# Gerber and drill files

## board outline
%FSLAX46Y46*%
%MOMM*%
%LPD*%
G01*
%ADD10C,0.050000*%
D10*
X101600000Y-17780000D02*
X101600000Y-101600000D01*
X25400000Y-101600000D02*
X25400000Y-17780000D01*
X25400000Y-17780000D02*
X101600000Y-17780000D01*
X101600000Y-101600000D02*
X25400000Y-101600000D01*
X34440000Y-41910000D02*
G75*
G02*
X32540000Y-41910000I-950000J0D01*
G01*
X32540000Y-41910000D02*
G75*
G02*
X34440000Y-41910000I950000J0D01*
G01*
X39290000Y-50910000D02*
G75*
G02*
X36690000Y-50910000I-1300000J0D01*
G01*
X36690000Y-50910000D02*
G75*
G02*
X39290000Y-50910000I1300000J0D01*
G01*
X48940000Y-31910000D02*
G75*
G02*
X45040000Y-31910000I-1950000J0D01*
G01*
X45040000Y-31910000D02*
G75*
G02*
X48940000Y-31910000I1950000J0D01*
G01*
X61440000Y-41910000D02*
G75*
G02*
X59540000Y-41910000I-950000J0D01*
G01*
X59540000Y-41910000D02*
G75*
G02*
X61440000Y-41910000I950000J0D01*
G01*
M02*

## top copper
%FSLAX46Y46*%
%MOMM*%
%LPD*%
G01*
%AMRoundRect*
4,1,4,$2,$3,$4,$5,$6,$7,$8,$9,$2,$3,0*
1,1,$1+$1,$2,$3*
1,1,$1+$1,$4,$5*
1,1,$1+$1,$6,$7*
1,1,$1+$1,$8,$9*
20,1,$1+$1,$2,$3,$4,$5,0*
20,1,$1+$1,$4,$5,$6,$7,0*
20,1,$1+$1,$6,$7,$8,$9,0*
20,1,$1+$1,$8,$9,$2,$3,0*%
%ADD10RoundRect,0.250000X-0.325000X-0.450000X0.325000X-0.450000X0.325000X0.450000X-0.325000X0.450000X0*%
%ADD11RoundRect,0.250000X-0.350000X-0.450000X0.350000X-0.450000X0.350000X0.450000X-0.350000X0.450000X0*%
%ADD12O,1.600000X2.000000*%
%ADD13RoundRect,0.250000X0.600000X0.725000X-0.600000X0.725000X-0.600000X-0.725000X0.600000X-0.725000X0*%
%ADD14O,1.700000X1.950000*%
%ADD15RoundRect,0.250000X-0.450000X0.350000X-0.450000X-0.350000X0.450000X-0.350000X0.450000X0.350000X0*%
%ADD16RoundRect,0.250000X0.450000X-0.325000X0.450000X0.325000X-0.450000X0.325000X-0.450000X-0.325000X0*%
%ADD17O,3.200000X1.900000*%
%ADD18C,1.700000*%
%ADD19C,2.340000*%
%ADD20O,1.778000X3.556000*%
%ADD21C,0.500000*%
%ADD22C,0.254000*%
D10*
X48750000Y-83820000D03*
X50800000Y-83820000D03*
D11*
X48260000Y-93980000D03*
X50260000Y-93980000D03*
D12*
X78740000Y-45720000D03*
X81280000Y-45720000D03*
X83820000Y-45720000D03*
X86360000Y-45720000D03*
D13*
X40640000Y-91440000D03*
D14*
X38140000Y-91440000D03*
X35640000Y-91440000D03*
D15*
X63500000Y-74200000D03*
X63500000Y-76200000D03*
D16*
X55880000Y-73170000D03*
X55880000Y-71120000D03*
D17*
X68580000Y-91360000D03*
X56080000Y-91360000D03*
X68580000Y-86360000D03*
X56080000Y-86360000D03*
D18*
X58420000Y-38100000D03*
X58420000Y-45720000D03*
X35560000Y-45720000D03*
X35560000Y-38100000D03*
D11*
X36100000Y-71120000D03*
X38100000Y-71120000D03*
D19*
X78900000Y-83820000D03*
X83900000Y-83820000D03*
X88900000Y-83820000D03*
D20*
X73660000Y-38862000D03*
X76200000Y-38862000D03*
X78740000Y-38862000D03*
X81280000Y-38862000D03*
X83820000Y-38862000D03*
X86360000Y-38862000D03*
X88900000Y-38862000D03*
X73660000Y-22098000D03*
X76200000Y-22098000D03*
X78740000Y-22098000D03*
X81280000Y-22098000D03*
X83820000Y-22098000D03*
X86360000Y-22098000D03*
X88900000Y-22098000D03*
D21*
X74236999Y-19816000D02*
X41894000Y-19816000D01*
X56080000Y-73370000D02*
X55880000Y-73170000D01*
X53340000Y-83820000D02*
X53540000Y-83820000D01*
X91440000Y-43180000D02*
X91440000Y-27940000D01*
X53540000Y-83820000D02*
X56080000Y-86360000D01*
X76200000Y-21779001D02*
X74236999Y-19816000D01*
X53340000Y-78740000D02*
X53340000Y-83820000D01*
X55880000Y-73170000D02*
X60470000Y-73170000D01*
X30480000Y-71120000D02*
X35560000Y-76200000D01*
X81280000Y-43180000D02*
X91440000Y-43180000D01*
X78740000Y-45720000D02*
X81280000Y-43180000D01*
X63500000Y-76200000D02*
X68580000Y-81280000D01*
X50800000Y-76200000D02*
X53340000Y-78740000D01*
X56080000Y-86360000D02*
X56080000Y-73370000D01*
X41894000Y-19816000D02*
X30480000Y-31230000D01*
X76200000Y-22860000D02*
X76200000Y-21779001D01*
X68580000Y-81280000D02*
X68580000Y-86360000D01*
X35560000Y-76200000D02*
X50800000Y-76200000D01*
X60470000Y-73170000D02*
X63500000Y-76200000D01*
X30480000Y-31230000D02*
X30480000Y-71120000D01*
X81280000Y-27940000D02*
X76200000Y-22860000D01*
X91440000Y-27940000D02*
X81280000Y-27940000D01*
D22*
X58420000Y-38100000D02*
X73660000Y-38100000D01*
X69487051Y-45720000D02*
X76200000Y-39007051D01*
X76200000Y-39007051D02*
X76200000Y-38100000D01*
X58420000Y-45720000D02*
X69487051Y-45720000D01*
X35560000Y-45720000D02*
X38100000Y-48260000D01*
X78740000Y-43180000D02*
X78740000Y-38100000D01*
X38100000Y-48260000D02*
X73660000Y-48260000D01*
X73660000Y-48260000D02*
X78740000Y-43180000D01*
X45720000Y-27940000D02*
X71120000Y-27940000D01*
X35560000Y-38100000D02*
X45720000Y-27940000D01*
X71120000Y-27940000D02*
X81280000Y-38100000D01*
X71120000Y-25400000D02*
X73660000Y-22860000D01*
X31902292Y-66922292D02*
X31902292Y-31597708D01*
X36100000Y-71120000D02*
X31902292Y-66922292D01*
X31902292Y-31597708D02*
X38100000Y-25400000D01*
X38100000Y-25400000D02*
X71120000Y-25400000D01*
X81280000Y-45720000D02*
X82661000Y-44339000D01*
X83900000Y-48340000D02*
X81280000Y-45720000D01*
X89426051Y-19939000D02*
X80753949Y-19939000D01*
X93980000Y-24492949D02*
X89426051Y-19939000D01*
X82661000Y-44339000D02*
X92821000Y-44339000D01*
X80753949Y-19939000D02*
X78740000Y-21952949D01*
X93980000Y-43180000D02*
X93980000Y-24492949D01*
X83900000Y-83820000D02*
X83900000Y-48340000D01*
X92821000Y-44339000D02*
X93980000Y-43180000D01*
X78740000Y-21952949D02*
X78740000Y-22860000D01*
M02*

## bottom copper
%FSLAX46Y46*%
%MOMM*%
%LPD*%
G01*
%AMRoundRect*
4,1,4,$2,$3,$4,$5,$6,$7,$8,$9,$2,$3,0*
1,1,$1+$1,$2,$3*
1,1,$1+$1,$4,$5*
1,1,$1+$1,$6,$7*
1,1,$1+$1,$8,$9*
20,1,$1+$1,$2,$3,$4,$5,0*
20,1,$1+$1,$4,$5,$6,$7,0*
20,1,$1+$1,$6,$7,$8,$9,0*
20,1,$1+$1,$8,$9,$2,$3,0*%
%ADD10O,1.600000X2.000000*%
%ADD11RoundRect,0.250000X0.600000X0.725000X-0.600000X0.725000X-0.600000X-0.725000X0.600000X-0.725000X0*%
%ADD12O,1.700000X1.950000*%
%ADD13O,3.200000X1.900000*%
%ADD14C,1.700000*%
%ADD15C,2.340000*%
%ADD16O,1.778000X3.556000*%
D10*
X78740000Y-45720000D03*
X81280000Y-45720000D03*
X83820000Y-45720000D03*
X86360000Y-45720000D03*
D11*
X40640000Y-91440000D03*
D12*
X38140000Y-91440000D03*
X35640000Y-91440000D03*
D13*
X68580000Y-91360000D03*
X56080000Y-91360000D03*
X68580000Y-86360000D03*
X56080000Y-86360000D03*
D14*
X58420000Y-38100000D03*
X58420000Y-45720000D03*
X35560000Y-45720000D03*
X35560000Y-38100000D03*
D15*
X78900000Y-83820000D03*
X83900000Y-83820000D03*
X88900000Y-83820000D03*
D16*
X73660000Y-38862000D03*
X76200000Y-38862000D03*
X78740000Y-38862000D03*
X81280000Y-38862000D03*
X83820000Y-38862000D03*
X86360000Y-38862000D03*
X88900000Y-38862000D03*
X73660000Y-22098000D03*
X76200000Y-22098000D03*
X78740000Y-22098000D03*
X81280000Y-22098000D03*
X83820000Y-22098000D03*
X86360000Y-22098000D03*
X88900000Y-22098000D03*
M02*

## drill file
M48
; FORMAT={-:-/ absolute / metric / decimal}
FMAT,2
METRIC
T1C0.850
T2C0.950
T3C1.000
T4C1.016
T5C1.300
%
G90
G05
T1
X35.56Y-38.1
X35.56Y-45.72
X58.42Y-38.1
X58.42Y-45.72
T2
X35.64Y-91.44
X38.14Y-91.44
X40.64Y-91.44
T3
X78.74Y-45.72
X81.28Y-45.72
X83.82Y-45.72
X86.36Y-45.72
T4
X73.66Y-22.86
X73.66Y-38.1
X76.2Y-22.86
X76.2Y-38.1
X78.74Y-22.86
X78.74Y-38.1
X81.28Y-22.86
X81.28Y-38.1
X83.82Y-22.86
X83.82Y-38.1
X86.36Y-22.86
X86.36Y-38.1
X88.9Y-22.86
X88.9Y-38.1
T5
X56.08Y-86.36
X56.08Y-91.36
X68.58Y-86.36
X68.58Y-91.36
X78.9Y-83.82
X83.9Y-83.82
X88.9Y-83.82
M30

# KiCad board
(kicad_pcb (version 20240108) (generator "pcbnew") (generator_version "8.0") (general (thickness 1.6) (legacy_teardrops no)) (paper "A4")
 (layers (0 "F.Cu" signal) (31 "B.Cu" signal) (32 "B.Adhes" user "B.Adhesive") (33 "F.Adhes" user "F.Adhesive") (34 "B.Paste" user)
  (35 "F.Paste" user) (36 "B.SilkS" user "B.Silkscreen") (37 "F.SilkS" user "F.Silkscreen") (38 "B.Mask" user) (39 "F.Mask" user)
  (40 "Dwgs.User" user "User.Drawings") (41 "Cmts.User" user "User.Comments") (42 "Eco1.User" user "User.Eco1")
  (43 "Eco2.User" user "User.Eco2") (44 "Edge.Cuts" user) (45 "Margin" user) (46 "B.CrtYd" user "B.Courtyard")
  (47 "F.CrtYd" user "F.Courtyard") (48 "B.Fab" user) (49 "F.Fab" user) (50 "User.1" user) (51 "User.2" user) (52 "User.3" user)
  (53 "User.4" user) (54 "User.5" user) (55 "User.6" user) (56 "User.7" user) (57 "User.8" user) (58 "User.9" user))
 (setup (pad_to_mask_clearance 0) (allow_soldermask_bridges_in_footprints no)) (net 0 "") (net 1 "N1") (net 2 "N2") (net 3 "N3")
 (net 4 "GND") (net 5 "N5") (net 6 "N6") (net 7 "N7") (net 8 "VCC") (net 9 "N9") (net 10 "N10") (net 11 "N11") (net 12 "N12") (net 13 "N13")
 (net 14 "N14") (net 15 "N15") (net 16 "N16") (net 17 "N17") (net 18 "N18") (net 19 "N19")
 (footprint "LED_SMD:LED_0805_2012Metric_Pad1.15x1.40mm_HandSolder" (layer "F.Cu") (at 49.775 83.82)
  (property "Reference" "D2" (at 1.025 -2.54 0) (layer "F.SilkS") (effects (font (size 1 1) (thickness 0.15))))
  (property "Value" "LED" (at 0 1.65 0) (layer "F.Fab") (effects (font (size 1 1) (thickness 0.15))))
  (pad "1" smd roundrect (at -1.025 0) (size 1.15 1.4) (layers "F.Cu" "F.Paste" "F.Mask") (roundrect_rratio 0.217391) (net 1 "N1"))
  (pad "2" smd roundrect (at 1.025 0) (size 1.15 1.4) (layers "F.Cu" "F.Paste" "F.Mask") (roundrect_rratio 0.217391) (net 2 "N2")))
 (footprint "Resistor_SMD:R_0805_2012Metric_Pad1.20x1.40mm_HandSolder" (layer "F.Cu") (at 49.26 93.98)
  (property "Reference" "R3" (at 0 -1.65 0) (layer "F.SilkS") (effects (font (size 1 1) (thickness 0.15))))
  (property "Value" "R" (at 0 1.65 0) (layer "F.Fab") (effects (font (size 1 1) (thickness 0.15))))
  (pad "1" smd roundrect (at -1 0) (size 1.2 1.4) (layers "F.Cu" "F.Paste" "F.Mask") (roundrect_rratio 0.208333) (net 1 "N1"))
  (pad "2" smd roundrect (at 1 0) (size 1.2 1.4) (layers "F.Cu" "F.Paste" "F.Mask") (roundrect_rratio 0.208333) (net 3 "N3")))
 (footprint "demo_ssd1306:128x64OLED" (layer "F.Cu") (at 82.36 56.32)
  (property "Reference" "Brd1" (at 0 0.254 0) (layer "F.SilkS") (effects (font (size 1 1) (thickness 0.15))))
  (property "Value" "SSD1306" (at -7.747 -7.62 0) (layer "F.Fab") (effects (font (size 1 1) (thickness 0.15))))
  (pad "1" thru_hole oval (at -3.62 -10.6 90) (size 2 1.6) (drill 1) (layers "*.Cu" "*.Mask") (remove_unused_layers no) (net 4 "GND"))
  (pad "2" thru_hole oval (at -1.08 -10.6 90) (size 2 1.6) (drill 1) (layers "*.Cu" "*.Mask") (remove_unused_layers no) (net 2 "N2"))
  (pad "3" thru_hole oval (at 1.46 -10.6 90) (size 2 1.6) (drill 1) (layers "*.Cu" "*.Mask") (remove_unused_layers no) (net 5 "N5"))
  (pad "4" thru_hole oval (at 4 -10.6 90) (size 2 1.6) (drill 1) (layers "*.Cu" "*.Mask") (remove_unused_layers no) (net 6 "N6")))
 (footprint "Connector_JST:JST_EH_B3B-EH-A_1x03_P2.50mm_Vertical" (layer "F.Cu") (at 40.64 91.44 180)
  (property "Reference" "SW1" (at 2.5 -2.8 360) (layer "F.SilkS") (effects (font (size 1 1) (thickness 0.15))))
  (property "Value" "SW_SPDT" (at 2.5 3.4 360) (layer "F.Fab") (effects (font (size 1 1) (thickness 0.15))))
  (pad "1" thru_hole roundrect (at 0 0 180) (size 1.7 1.95) (drill 0.95) (layers "*.Cu" "*.Mask") (remove_unused_layers no)
   (roundrect_rratio 0.147059) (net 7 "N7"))
  (pad "2" thru_hole oval (at 2.5 0 180) (size 1.7 1.95) (drill 0.95) (layers "*.Cu" "*.Mask") (remove_unused_layers no) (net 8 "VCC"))
  (pad "3" thru_hole oval (at 5 0 180) (size 1.7 1.95) (drill 0.95) (layers "*.Cu" "*.Mask") (remove_unused_layers no) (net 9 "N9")))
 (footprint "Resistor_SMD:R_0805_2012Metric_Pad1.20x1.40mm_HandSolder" (layer "F.Cu") (at 63.5 75.2 -90)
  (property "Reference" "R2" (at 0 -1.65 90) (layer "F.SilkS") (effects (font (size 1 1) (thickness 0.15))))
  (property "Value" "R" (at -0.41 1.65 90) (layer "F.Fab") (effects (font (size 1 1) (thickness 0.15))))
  (pad "1" smd roundrect (at -1 0 270) (size 1.2 1.4) (layers "F.Cu" "F.Paste" "F.Mask") (roundrect_rratio 0.208333) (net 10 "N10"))
  (pad "2" smd roundrect (at 1 0 270) (size 1.2 1.4) (layers "F.Cu" "F.Paste" "F.Mask") (roundrect_rratio 0.208333) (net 4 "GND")))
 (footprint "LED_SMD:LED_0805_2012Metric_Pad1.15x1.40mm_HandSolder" (layer "F.Cu") (at 55.88 72.145 90)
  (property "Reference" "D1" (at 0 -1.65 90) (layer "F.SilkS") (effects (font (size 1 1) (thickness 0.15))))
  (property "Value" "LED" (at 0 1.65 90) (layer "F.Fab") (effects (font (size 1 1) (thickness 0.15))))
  (pad "1" smd roundrect (at -1.025 0 90) (size 1.15 1.4) (layers "F.Cu" "F.Paste" "F.Mask") (roundrect_rratio 0.217391) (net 4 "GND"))
  (pad "2" smd roundrect (at 1.025 0 90) (size 1.15 1.4) (layers "F.Cu" "F.Paste" "F.Mask") (roundrect_rratio 0.217391) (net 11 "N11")))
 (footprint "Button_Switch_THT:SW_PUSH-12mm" (layer "F.Cu") (at 68.58 91.36 180)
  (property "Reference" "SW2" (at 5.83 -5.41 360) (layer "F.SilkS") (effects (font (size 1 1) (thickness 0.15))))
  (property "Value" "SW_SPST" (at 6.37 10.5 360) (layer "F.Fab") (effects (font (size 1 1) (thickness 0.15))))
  (pad "1" thru_hole oval (at 0 0 180) (size 3.2 1.9) (drill 1.3) (layers "*.Cu" "*.Mask") (remove_unused_layers no) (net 3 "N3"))
  (pad "1" thru_hole oval (at 12.5 0 180) (size 3.2 1.9) (drill 1.3) (layers "*.Cu" "*.Mask") (remove_unused_layers no) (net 3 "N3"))
  (pad "2" thru_hole oval (at 0 5 180) (size 3.2 1.9) (drill 1.3) (layers "*.Cu" "*.Mask") (remove_unused_layers no) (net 4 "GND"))
  (pad "2" thru_hole oval (at 12.5 5 180) (size 3.2 1.9) (drill 1.3) (layers "*.Cu" "*.Mask") (remove_unused_layers no) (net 4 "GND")))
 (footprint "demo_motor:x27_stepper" (layer "F.Cu") (at 49.53 52.07)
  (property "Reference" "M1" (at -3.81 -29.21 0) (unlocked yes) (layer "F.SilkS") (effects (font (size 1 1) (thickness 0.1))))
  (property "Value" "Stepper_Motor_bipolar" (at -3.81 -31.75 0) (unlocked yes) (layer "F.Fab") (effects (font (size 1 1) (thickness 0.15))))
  (fp_circle (center -16.04 -10.16) (end -15.09 -10.16) (stroke (width 0.05) (type default)) (fill none) (layer "Edge.Cuts"))
  (fp_circle (center -11.54 -1.16) (end -10.24 -1.16) (stroke (width 0.05) (type default)) (fill none) (layer "Edge.Cuts"))
  (fp_circle (center -2.54 -20.16) (end -0.59 -20.16) (stroke (width 0.05) (type default)) (fill none) (layer "Edge.Cuts"))
  (fp_circle (center 10.96 -10.16) (end 11.91 -10.16) (stroke (width 0.05) (type default)) (fill none) (layer "Edge.Cuts"))
  (pad "1" thru_hole circle (at 8.89 -13.97) (size 1.7 1.7) (drill 0.85) (layers "*.Cu" "*.Mask") (remove_unused_layers no) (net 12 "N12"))
  (pad "2" thru_hole circle (at 8.89 -6.35) (size 1.7 1.7) (drill 0.85) (layers "*.Cu" "*.Mask") (remove_unused_layers no) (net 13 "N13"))
  (pad "3" thru_hole circle (at -13.97 -6.35) (size 1.7 1.7) (drill 0.85) (layers "*.Cu" "*.Mask") (remove_unused_layers no) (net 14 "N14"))
  (pad "4" thru_hole circle (at -13.97 -13.97) (size 1.7 1.7) (drill 0.85) (layers "*.Cu" "*.Mask") (remove_unused_layers no) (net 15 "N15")))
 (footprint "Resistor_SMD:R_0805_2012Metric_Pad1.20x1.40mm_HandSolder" (layer "F.Cu") (at 37.1 71.12)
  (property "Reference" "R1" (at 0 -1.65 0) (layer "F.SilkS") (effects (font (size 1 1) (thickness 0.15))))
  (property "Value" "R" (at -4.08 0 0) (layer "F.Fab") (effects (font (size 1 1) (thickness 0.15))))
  (pad "1" smd roundrect (at -1 0) (size 1.2 1.4) (layers "F.Cu" "F.Paste" "F.Mask") (roundrect_rratio 0.208333) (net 9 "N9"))
  (pad "2" smd roundrect (at 1 0) (size 1.2 1.4) (layers "F.Cu" "F.Paste" "F.Mask") (roundrect_rratio 0.208333) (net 11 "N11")))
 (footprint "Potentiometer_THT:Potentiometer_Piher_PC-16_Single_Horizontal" (layer "F.Cu") (at 78.9 83.82 -90)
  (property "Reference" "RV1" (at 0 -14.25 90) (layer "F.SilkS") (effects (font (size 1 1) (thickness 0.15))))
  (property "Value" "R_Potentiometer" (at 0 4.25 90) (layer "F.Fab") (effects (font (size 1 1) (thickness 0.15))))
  (pad "1" thru_hole circle (at 0 0 270) (size 2.34 2.34) (drill 1.3) (layers "*.Cu" "*.Mask") (remove_unused_layers no) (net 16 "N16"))
  (pad "2" thru_hole circle (at 0 -5 270) (size 2.34 2.34) (drill 1.3) (layers "*.Cu" "*.Mask") (remove_unused_layers no) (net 2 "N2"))
  (pad "3" thru_hole circle (at 0 -10 270) (size 2.34 2.34) (drill 1.3) (layers "*.Cu" "*.Mask") (remove_unused_layers no) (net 10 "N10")))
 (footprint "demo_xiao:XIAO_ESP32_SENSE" (layer "F.Cu") (at 81.28 30.48 90)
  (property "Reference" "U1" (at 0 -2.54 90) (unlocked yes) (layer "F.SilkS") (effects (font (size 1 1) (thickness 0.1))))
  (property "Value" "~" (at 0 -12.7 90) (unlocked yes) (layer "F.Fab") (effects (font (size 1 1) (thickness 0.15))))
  (pad "1" thru_hole oval (at -7.62 -7.62 90) (size 3.556 1.778) (drill 1.016 (offset -0.762 0)) (layers "*.Cu" "*.Mask")
   (remove_unused_layers no) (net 12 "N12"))
  (pad "2" thru_hole oval (at -7.62 -5.08 90) (size 3.556 1.778) (drill 1.016 (offset -0.762 0)) (layers "*.Cu" "*.Mask")
   (remove_unused_layers no) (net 13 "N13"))
  (pad "3" thru_hole oval (at -7.62 -2.54 90) (size 3.556 1.778) (drill 1.016 (offset -0.762 0)) (layers "*.Cu" "*.Mask")
   (remove_unused_layers no) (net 14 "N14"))
  (pad "4" thru_hole oval (at -7.62 0 90) (size 3.556 1.778) (drill 1.016 (offset -0.762 0)) (layers "*.Cu" "*.Mask")
   (remove_unused_layers no) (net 15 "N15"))
  (pad "5" thru_hole oval (at -7.62 2.54 90) (size 3.556 1.778) (drill 1.016 (offset -0.762 0)) (layers "*.Cu" "*.Mask")
   (remove_unused_layers no) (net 6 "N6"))
  (pad "6" thru_hole oval (at -7.62 5.08 90) (size 3.556 1.778) (drill 1.016 (offset -0.762 0)) (layers "*.Cu" "*.Mask")
   (remove_unused_layers no) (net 5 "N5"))
  (pad "7" thru_hole oval (at -7.62 7.62 90) (size 3.556 1.778) (drill 1.016 (offset -0.762 0)) (layers "*.Cu" "*.Mask")
   (remove_unused_layers no) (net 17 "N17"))
  (pad "8" thru_hole oval (at 7.62 -7.62 90) (size 3.556 1.778) (drill 1.016 (offset 0.762 0)) (layers "*.Cu" "*.Mask")
   (remove_unused_layers no) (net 9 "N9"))
  (pad "9" thru_hole oval (at 7.62 -5.08 90) (size 3.556 1.778) (drill 1.016 (offset 0.762 0)) (layers "*.Cu" "*.Mask")
   (remove_unused_layers no) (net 4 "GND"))
  (pad "10" thru_hole oval (at 7.62 -2.54 90) (size 3.556 1.778) (drill 1.016 (offset 0.762 0)) (layers "*.Cu" "*.Mask")
   (remove_unused_layers no) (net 2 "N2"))
  (pad "11" thru_hole oval (at 7.62 0 90) (size 3.556 1.778) (drill 1.016 (offset 0.762 0)) (layers "*.Cu" "*.Mask")
   (remove_unused_layers no) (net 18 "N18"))
  (pad "12" thru_hole oval (at 7.62 2.54 90) (size 3.556 1.778) (drill 1.016 (offset 0.762 0)) (layers "*.Cu" "*.Mask")
   (remove_unused_layers no) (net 10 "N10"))
  (pad "13" thru_hole oval (at 7.62 5.08 90) (size 3.556 1.778) (drill 1.016 (offset 0.762 0)) (layers "*.Cu" "*.Mask")
   (remove_unused_layers no) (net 3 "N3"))
  (pad "14" thru_hole oval (at 7.62 7.62 90) (size 3.556 1.778) (drill 1.016 (offset 0.762 0)) (layers "*.Cu" "*.Mask")
   (remove_unused_layers no) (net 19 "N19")))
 (gr_line (start 101.6 17.78) (end 101.6 101.6) (stroke (width 0.05) (type default)) (layer "Edge.Cuts"))
 (gr_line (start 25.4 101.6) (end 25.4 17.78) (stroke (width 0.05) (type default)) (layer "Edge.Cuts"))
 (gr_line (start 25.4 17.78) (end 101.6 17.78) (stroke (width 0.05) (type default)) (layer "Edge.Cuts"))
 (gr_line (start 101.6 101.6) (end 25.4 101.6) (stroke (width 0.05) (type default)) (layer "Edge.Cuts"))
 (segment (start 74.236999 19.816) (end 41.894 19.816) (width 0.5) (layer "F.Cu") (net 4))
 (segment (start 56.08 73.37) (end 55.88 73.17) (width 0.5) (layer "F.Cu") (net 4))
 (segment (start 53.34 83.82) (end 53.54 83.82) (width 0.5) (layer "F.Cu") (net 4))
 (segment (start 91.44 43.18) (end 91.44 27.94) (width 0.5) (layer "F.Cu") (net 4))
 (segment (start 53.54 83.82) (end 56.08 86.36) (width 0.5) (layer "F.Cu") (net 4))
 (segment (start 76.2 21.779001) (end 74.236999 19.816) (width 0.5) (layer "F.Cu") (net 4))
 (segment (start 53.34 78.74) (end 53.34 83.82) (width 0.5) (layer "F.Cu") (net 4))
 (segment (start 55.88 73.17) (end 60.47 73.17) (width 0.5) (layer "F.Cu") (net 4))
 (segment (start 30.48 71.12) (end 35.56 76.2) (width 0.5) (layer "F.Cu") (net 4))
 (segment (start 81.28 43.18) (end 91.44 43.18) (width 0.5) (layer "F.Cu") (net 4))
 (segment (start 78.74 45.72) (end 81.28 43.18) (width 0.5) (layer "F.Cu") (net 4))
 (segment (start 63.5 76.2) (end 68.58 81.28) (width 0.5) (layer "F.Cu") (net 4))
 (segment (start 50.8 76.2) (end 53.34 78.74) (width 0.5) (layer "F.Cu") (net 4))
 (segment (start 56.08 86.36) (end 56.08 73.37) (width 0.5) (layer "F.Cu") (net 4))
 (segment (start 41.894 19.816) (end 30.48 31.23) (width 0.5) (layer "F.Cu") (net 4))
 (segment (start 76.2 22.86) (end 76.2 21.779001) (width 0.5) (layer "F.Cu") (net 4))
 (segment (start 68.58 81.28) (end 68.58 86.36) (width 0.5) (layer "F.Cu") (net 4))
 (segment (start 35.56 76.2) (end 50.8 76.2) (width 0.5) (layer "F.Cu") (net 4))
 (segment (start 60.47 73.17) (end 63.5 76.2) (width 0.5) (layer "F.Cu") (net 4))
 (segment (start 30.48 31.23) (end 30.48 71.12) (width 0.5) (layer "F.Cu") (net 4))
 (segment (start 81.28 27.94) (end 76.2 22.86) (width 0.5) (layer "F.Cu") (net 4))
 (segment (start 91.44 27.94) (end 81.28 27.94) (width 0.5) (layer "F.Cu") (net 4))
 (segment (start 58.42 38.1) (end 73.66 38.1) (width 0.254) (layer "F.Cu") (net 12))
 (segment (start 69.487051 45.72) (end 76.2 39.007051) (width 0.254) (layer "F.Cu") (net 13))
 (segment (start 76.2 39.007051) (end 76.2 38.1) (width 0.254) (layer "F.Cu") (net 13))
 (segment (start 58.42 45.72) (end 69.487051 45.72) (width 0.254) (layer "F.Cu") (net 13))
 (segment (start 35.56 45.72) (end 38.1 48.26) (width 0.254) (layer "F.Cu") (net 14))
 (segment (start 78.74 43.18) (end 78.74 38.1) (width 0.254) (layer "F.Cu") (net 14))
 (segment (start 38.1 48.26) (end 73.66 48.26) (width 0.254) (layer "F.Cu") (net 14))
 (segment (start 73.66 48.26) (end 78.74 43.18) (width 0.254) (layer "F.Cu") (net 14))
 (segment (start 45.72 27.94) (end 71.12 27.94) (width 0.254) (layer "F.Cu") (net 15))
 (segment (start 35.56 38.1) (end 45.72 27.94) (width 0.254) (layer "F.Cu") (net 15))
 (segment (start 71.12 27.94) (end 81.28 38.1) (width 0.254) (layer "F.Cu") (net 15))
 (segment (start 71.12 25.4) (end 73.66 22.86) (width 0.254) (layer "F.Cu") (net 9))
 (segment (start 31.902292 66.922292) (end 31.902292 31.597708) (width 0.254) (layer "F.Cu") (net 9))
 (segment (start 36.1 71.12) (end 31.902292 66.922292) (width 0.254) (layer "F.Cu") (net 9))
 (segment (start 31.902292 31.597708) (end 38.1 25.4) (width 0.254) (layer "F.Cu") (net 9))
 (segment (start 38.1 25.4) (end 71.12 25.4) (width 0.254) (layer "F.Cu") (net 9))
 (segment (start 81.28 45.72) (end 82.661 44.339) (width 0.254) (layer "F.Cu") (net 2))
 (segment (start 83.9 48.34) (end 81.28 45.72) (width 0.254) (layer "F.Cu") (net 2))
 (segment (start 89.426051 19.939) (end 80.753949 19.939) (width 0.254) (layer "F.Cu") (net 2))
 (segment (start 93.98 24.492949) (end 89.426051 19.939) (width 0.254) (layer "F.Cu") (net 2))
 (segment (start 82.661 44.339) (end 92.821 44.339) (width 0.254) (layer "F.Cu") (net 2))
 (segment (start 80.753949 19.939) (end 78.74 21.952949) (width 0.254) (layer "F.Cu") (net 2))
 (segment (start 93.98 43.18) (end 93.98 24.492949) (width 0.254) (layer "F.Cu") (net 2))
 (segment (start 83.9 83.82) (end 83.9 48.34) (width 0.254) (layer "F.Cu") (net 2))
 (segment (start 92.821 44.339) (end 93.98 43.18) (width 0.254) (layer "F.Cu") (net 2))
 (segment (start 78.74 21.952949) (end 78.74 22.86) (width 0.254) (layer "F.Cu") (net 2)))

